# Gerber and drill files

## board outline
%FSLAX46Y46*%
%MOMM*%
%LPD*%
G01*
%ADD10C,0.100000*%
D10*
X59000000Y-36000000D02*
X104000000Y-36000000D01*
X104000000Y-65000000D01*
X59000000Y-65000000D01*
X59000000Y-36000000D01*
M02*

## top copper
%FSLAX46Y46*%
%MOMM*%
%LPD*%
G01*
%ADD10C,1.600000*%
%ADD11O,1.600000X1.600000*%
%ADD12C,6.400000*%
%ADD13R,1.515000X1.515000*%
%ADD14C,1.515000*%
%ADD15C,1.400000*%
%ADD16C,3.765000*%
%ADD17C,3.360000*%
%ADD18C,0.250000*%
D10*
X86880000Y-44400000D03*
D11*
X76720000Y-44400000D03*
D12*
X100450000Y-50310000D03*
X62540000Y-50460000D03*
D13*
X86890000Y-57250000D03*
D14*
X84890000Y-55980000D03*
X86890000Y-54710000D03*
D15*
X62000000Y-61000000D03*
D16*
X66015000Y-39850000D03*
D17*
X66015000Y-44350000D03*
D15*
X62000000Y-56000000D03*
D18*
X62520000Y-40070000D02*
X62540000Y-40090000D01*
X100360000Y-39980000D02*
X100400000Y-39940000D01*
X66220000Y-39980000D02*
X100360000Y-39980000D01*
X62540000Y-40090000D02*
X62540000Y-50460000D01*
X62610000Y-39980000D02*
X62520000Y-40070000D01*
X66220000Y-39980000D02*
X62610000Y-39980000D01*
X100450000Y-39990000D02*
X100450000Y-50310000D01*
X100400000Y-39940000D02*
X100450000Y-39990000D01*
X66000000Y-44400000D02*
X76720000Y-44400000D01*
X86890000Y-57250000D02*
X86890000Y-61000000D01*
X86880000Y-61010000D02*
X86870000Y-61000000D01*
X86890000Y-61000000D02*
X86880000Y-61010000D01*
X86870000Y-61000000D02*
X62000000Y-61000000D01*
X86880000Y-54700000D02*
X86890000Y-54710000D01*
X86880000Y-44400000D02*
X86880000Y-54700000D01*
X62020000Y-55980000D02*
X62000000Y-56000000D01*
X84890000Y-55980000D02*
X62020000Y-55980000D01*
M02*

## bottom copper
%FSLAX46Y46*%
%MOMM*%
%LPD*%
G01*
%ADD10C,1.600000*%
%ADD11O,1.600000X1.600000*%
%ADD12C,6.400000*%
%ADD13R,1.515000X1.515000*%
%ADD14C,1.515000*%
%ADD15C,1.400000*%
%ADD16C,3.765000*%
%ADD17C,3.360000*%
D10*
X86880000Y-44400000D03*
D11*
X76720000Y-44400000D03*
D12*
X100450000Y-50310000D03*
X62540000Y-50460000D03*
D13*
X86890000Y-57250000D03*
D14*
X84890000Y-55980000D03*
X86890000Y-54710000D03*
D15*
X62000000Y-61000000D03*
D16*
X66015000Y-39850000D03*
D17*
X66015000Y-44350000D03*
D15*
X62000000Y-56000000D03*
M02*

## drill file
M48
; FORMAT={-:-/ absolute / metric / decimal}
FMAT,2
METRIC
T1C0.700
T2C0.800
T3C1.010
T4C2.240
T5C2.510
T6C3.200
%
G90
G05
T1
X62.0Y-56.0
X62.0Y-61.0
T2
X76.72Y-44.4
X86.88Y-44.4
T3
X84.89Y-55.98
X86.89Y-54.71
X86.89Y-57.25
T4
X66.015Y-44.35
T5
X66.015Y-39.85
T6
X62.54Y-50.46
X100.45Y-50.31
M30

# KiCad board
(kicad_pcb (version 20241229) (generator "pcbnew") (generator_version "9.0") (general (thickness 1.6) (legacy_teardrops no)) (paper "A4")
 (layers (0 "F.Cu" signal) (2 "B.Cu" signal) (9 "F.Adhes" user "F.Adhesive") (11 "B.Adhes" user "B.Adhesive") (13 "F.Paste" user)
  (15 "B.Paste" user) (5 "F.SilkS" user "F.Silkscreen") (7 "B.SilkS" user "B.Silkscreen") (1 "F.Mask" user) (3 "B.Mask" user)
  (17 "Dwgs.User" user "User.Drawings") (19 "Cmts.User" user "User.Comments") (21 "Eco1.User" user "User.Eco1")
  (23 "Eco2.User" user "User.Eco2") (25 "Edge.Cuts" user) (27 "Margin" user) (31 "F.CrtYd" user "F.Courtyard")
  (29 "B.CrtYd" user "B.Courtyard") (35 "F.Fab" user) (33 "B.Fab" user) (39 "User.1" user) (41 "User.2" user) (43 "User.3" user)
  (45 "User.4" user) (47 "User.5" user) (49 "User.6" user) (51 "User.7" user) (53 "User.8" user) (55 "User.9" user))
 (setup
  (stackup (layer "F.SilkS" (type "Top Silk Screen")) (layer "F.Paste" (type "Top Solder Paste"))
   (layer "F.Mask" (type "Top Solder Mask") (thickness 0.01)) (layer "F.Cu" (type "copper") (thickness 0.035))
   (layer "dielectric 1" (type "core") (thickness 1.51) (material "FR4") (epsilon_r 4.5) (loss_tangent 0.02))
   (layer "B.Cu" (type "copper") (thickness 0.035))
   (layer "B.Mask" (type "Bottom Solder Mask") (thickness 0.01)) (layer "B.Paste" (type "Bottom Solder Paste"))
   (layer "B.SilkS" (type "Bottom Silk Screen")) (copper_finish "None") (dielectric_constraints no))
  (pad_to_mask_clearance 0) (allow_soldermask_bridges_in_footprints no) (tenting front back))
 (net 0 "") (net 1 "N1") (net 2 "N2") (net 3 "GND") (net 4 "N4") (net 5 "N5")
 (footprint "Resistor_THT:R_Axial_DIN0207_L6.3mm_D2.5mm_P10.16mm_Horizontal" (layer "F.Cu") (at 86.88 44.4 180)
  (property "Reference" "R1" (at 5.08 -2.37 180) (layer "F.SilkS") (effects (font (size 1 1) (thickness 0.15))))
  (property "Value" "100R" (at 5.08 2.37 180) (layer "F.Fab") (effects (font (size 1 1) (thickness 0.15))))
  (pad "1" thru_hole circle (at 0 0 180) (size 1.6 1.6) (drill 0.8) (layers "*.Cu" "*.Mask") (remove_unused_layers no) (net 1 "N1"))
  (pad "2" thru_hole oval (at 10.16 0 180) (size 1.6 1.6) (drill 0.8) (layers "*.Cu" "*.Mask") (remove_unused_layers no) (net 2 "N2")))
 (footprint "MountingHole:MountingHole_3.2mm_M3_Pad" (layer "F.Cu") (at 100.45 50.31)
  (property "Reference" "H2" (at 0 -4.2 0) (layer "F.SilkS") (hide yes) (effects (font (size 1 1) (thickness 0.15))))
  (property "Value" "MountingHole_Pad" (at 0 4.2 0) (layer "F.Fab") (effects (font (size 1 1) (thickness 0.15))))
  (pad "1" thru_hole circle (at 0 0) (size 6.4 6.4) (drill 3.2) (layers "*.Cu" "*.Mask") (remove_unused_layers no) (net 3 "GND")))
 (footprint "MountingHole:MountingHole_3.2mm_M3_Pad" (layer "F.Cu") (at 62.54 50.46)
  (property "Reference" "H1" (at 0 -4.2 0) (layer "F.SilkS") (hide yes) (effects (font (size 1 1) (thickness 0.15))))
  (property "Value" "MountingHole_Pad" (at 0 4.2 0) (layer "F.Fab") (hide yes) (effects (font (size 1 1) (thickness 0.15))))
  (pad "1" thru_hole circle (at 0 0) (size 6.4 6.4) (drill 3.2) (layers "*.Cu" "*.Mask") (remove_unused_layers no) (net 3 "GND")))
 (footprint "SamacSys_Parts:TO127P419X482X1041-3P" (layer "F.Cu") (at 86.89 57.25 90)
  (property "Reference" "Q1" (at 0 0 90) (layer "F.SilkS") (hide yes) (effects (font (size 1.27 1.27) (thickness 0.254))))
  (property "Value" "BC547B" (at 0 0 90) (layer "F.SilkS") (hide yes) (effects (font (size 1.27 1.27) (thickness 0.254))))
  (pad "1" thru_hole rect (at 0 0 90) (size 1.515 1.515) (drill 1.01) (layers "*.Cu" "*.Mask") (remove_unused_layers no) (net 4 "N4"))
  (pad "2" thru_hole circle (at 1.27 -2 90) (size 1.515 1.515) (drill 1.01) (layers "*.Cu" "*.Mask") (remove_unused_layers no) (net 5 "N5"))
  (pad "3" thru_hole circle (at 2.54 0 90) (size 1.515 1.515) (drill 1.01) (layers "*.Cu" "*.Mask") (remove_unused_layers no) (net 1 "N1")))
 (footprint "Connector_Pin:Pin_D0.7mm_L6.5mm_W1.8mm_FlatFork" (layer "F.Cu") (at 62 61)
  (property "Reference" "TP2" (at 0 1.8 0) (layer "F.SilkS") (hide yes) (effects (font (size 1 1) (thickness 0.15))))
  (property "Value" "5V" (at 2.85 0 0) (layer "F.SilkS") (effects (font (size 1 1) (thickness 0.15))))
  (pad "1" thru_hole circle (at 0 0) (size 1.4 1.4) (drill 0.7) (layers "*.Cu" "*.Mask") (remove_unused_layers no) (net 4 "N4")))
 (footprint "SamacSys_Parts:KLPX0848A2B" (layer "F.Cu") (at 66.015 39.85 -90)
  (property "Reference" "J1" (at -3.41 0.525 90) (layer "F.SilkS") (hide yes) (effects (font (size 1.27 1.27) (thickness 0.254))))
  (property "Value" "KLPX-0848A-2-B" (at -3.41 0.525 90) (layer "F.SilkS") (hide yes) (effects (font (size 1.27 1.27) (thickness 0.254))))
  (pad "1" thru_hole circle (at 0 0 270) (size 3.765 3.765) (drill 2.51) (layers "*.Cu" "*.Mask") (remove_unused_layers no) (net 3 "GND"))
  (pad "2" thru_hole circle (at 4.5 0 270) (size 3.36 3.36) (drill 2.24) (layers "*.Cu" "*.Mask") (remove_unused_layers no) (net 2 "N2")))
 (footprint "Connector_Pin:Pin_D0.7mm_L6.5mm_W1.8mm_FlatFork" (layer "F.Cu") (at 62 56)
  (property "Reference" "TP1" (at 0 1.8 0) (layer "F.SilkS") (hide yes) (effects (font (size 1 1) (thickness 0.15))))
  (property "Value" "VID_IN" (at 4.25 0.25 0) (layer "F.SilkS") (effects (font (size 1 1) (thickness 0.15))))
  (pad "1" thru_hole circle (at 0 0) (size 1.4 1.4) (drill 0.7) (layers "*.Cu" "*.Mask") (remove_unused_layers no) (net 5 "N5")))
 (gr_rect (start 59 36) (end 104 65) (stroke (width 0.1) (type default)) (fill no) (layer "Edge.Cuts"))
 (segment (start 62.52 40.07) (end 62.54 40.09) (width 0.25) (layer "F.Cu") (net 3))
 (segment (start 100.36 39.98) (end 100.4 39.94) (width 0.25) (layer "F.Cu") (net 3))
 (segment (start 66.22 39.98) (end 100.36 39.98) (width 0.25) (layer "F.Cu") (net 3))
 (segment (start 62.54 40.09) (end 62.54 50.46) (width 0.25) (layer "F.Cu") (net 3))
 (segment (start 62.61 39.98) (end 62.52 40.07) (width 0.25) (layer "F.Cu") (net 3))
 (segment (start 66.22 39.98) (end 62.61 39.98) (width 0.25) (layer "F.Cu") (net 3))
 (segment (start 100.45 39.99) (end 100.45 50.31) (width 0.25) (layer "F.Cu") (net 3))
 (segment (start 100.4 39.94) (end 100.45 39.99) (width 0.25) (layer "F.Cu") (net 3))
 (segment (start 66 44.4) (end 76.72 44.4) (width 0.25) (layer "F.Cu") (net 2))
 (segment (start 86.89 57.25) (end 86.89 61) (width 0.25) (layer "F.Cu") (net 4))
 (segment (start 86.88 61.01) (end 86.87 61) (width 0.25) (layer "F.Cu") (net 4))
 (segment (start 86.89 61) (end 86.88 61.01) (width 0.25) (layer "F.Cu") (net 4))
 (segment (start 86.87 61) (end 62 61) (width 0.25) (layer "F.Cu") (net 4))
 (segment (start 86.88 54.7) (end 86.89 54.71) (width 0.25) (layer "F.Cu") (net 1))
 (segment (start 86.88 44.4) (end 86.88 54.7) (width 0.25) (layer "F.Cu") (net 1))
 (segment (start 62.02 55.98) (end 62 56) (width 0.25) (layer "F.Cu") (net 5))
 (segment (start 84.89 55.98) (end 62.02 55.98) (width 0.25) (layer "F.Cu") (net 5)))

